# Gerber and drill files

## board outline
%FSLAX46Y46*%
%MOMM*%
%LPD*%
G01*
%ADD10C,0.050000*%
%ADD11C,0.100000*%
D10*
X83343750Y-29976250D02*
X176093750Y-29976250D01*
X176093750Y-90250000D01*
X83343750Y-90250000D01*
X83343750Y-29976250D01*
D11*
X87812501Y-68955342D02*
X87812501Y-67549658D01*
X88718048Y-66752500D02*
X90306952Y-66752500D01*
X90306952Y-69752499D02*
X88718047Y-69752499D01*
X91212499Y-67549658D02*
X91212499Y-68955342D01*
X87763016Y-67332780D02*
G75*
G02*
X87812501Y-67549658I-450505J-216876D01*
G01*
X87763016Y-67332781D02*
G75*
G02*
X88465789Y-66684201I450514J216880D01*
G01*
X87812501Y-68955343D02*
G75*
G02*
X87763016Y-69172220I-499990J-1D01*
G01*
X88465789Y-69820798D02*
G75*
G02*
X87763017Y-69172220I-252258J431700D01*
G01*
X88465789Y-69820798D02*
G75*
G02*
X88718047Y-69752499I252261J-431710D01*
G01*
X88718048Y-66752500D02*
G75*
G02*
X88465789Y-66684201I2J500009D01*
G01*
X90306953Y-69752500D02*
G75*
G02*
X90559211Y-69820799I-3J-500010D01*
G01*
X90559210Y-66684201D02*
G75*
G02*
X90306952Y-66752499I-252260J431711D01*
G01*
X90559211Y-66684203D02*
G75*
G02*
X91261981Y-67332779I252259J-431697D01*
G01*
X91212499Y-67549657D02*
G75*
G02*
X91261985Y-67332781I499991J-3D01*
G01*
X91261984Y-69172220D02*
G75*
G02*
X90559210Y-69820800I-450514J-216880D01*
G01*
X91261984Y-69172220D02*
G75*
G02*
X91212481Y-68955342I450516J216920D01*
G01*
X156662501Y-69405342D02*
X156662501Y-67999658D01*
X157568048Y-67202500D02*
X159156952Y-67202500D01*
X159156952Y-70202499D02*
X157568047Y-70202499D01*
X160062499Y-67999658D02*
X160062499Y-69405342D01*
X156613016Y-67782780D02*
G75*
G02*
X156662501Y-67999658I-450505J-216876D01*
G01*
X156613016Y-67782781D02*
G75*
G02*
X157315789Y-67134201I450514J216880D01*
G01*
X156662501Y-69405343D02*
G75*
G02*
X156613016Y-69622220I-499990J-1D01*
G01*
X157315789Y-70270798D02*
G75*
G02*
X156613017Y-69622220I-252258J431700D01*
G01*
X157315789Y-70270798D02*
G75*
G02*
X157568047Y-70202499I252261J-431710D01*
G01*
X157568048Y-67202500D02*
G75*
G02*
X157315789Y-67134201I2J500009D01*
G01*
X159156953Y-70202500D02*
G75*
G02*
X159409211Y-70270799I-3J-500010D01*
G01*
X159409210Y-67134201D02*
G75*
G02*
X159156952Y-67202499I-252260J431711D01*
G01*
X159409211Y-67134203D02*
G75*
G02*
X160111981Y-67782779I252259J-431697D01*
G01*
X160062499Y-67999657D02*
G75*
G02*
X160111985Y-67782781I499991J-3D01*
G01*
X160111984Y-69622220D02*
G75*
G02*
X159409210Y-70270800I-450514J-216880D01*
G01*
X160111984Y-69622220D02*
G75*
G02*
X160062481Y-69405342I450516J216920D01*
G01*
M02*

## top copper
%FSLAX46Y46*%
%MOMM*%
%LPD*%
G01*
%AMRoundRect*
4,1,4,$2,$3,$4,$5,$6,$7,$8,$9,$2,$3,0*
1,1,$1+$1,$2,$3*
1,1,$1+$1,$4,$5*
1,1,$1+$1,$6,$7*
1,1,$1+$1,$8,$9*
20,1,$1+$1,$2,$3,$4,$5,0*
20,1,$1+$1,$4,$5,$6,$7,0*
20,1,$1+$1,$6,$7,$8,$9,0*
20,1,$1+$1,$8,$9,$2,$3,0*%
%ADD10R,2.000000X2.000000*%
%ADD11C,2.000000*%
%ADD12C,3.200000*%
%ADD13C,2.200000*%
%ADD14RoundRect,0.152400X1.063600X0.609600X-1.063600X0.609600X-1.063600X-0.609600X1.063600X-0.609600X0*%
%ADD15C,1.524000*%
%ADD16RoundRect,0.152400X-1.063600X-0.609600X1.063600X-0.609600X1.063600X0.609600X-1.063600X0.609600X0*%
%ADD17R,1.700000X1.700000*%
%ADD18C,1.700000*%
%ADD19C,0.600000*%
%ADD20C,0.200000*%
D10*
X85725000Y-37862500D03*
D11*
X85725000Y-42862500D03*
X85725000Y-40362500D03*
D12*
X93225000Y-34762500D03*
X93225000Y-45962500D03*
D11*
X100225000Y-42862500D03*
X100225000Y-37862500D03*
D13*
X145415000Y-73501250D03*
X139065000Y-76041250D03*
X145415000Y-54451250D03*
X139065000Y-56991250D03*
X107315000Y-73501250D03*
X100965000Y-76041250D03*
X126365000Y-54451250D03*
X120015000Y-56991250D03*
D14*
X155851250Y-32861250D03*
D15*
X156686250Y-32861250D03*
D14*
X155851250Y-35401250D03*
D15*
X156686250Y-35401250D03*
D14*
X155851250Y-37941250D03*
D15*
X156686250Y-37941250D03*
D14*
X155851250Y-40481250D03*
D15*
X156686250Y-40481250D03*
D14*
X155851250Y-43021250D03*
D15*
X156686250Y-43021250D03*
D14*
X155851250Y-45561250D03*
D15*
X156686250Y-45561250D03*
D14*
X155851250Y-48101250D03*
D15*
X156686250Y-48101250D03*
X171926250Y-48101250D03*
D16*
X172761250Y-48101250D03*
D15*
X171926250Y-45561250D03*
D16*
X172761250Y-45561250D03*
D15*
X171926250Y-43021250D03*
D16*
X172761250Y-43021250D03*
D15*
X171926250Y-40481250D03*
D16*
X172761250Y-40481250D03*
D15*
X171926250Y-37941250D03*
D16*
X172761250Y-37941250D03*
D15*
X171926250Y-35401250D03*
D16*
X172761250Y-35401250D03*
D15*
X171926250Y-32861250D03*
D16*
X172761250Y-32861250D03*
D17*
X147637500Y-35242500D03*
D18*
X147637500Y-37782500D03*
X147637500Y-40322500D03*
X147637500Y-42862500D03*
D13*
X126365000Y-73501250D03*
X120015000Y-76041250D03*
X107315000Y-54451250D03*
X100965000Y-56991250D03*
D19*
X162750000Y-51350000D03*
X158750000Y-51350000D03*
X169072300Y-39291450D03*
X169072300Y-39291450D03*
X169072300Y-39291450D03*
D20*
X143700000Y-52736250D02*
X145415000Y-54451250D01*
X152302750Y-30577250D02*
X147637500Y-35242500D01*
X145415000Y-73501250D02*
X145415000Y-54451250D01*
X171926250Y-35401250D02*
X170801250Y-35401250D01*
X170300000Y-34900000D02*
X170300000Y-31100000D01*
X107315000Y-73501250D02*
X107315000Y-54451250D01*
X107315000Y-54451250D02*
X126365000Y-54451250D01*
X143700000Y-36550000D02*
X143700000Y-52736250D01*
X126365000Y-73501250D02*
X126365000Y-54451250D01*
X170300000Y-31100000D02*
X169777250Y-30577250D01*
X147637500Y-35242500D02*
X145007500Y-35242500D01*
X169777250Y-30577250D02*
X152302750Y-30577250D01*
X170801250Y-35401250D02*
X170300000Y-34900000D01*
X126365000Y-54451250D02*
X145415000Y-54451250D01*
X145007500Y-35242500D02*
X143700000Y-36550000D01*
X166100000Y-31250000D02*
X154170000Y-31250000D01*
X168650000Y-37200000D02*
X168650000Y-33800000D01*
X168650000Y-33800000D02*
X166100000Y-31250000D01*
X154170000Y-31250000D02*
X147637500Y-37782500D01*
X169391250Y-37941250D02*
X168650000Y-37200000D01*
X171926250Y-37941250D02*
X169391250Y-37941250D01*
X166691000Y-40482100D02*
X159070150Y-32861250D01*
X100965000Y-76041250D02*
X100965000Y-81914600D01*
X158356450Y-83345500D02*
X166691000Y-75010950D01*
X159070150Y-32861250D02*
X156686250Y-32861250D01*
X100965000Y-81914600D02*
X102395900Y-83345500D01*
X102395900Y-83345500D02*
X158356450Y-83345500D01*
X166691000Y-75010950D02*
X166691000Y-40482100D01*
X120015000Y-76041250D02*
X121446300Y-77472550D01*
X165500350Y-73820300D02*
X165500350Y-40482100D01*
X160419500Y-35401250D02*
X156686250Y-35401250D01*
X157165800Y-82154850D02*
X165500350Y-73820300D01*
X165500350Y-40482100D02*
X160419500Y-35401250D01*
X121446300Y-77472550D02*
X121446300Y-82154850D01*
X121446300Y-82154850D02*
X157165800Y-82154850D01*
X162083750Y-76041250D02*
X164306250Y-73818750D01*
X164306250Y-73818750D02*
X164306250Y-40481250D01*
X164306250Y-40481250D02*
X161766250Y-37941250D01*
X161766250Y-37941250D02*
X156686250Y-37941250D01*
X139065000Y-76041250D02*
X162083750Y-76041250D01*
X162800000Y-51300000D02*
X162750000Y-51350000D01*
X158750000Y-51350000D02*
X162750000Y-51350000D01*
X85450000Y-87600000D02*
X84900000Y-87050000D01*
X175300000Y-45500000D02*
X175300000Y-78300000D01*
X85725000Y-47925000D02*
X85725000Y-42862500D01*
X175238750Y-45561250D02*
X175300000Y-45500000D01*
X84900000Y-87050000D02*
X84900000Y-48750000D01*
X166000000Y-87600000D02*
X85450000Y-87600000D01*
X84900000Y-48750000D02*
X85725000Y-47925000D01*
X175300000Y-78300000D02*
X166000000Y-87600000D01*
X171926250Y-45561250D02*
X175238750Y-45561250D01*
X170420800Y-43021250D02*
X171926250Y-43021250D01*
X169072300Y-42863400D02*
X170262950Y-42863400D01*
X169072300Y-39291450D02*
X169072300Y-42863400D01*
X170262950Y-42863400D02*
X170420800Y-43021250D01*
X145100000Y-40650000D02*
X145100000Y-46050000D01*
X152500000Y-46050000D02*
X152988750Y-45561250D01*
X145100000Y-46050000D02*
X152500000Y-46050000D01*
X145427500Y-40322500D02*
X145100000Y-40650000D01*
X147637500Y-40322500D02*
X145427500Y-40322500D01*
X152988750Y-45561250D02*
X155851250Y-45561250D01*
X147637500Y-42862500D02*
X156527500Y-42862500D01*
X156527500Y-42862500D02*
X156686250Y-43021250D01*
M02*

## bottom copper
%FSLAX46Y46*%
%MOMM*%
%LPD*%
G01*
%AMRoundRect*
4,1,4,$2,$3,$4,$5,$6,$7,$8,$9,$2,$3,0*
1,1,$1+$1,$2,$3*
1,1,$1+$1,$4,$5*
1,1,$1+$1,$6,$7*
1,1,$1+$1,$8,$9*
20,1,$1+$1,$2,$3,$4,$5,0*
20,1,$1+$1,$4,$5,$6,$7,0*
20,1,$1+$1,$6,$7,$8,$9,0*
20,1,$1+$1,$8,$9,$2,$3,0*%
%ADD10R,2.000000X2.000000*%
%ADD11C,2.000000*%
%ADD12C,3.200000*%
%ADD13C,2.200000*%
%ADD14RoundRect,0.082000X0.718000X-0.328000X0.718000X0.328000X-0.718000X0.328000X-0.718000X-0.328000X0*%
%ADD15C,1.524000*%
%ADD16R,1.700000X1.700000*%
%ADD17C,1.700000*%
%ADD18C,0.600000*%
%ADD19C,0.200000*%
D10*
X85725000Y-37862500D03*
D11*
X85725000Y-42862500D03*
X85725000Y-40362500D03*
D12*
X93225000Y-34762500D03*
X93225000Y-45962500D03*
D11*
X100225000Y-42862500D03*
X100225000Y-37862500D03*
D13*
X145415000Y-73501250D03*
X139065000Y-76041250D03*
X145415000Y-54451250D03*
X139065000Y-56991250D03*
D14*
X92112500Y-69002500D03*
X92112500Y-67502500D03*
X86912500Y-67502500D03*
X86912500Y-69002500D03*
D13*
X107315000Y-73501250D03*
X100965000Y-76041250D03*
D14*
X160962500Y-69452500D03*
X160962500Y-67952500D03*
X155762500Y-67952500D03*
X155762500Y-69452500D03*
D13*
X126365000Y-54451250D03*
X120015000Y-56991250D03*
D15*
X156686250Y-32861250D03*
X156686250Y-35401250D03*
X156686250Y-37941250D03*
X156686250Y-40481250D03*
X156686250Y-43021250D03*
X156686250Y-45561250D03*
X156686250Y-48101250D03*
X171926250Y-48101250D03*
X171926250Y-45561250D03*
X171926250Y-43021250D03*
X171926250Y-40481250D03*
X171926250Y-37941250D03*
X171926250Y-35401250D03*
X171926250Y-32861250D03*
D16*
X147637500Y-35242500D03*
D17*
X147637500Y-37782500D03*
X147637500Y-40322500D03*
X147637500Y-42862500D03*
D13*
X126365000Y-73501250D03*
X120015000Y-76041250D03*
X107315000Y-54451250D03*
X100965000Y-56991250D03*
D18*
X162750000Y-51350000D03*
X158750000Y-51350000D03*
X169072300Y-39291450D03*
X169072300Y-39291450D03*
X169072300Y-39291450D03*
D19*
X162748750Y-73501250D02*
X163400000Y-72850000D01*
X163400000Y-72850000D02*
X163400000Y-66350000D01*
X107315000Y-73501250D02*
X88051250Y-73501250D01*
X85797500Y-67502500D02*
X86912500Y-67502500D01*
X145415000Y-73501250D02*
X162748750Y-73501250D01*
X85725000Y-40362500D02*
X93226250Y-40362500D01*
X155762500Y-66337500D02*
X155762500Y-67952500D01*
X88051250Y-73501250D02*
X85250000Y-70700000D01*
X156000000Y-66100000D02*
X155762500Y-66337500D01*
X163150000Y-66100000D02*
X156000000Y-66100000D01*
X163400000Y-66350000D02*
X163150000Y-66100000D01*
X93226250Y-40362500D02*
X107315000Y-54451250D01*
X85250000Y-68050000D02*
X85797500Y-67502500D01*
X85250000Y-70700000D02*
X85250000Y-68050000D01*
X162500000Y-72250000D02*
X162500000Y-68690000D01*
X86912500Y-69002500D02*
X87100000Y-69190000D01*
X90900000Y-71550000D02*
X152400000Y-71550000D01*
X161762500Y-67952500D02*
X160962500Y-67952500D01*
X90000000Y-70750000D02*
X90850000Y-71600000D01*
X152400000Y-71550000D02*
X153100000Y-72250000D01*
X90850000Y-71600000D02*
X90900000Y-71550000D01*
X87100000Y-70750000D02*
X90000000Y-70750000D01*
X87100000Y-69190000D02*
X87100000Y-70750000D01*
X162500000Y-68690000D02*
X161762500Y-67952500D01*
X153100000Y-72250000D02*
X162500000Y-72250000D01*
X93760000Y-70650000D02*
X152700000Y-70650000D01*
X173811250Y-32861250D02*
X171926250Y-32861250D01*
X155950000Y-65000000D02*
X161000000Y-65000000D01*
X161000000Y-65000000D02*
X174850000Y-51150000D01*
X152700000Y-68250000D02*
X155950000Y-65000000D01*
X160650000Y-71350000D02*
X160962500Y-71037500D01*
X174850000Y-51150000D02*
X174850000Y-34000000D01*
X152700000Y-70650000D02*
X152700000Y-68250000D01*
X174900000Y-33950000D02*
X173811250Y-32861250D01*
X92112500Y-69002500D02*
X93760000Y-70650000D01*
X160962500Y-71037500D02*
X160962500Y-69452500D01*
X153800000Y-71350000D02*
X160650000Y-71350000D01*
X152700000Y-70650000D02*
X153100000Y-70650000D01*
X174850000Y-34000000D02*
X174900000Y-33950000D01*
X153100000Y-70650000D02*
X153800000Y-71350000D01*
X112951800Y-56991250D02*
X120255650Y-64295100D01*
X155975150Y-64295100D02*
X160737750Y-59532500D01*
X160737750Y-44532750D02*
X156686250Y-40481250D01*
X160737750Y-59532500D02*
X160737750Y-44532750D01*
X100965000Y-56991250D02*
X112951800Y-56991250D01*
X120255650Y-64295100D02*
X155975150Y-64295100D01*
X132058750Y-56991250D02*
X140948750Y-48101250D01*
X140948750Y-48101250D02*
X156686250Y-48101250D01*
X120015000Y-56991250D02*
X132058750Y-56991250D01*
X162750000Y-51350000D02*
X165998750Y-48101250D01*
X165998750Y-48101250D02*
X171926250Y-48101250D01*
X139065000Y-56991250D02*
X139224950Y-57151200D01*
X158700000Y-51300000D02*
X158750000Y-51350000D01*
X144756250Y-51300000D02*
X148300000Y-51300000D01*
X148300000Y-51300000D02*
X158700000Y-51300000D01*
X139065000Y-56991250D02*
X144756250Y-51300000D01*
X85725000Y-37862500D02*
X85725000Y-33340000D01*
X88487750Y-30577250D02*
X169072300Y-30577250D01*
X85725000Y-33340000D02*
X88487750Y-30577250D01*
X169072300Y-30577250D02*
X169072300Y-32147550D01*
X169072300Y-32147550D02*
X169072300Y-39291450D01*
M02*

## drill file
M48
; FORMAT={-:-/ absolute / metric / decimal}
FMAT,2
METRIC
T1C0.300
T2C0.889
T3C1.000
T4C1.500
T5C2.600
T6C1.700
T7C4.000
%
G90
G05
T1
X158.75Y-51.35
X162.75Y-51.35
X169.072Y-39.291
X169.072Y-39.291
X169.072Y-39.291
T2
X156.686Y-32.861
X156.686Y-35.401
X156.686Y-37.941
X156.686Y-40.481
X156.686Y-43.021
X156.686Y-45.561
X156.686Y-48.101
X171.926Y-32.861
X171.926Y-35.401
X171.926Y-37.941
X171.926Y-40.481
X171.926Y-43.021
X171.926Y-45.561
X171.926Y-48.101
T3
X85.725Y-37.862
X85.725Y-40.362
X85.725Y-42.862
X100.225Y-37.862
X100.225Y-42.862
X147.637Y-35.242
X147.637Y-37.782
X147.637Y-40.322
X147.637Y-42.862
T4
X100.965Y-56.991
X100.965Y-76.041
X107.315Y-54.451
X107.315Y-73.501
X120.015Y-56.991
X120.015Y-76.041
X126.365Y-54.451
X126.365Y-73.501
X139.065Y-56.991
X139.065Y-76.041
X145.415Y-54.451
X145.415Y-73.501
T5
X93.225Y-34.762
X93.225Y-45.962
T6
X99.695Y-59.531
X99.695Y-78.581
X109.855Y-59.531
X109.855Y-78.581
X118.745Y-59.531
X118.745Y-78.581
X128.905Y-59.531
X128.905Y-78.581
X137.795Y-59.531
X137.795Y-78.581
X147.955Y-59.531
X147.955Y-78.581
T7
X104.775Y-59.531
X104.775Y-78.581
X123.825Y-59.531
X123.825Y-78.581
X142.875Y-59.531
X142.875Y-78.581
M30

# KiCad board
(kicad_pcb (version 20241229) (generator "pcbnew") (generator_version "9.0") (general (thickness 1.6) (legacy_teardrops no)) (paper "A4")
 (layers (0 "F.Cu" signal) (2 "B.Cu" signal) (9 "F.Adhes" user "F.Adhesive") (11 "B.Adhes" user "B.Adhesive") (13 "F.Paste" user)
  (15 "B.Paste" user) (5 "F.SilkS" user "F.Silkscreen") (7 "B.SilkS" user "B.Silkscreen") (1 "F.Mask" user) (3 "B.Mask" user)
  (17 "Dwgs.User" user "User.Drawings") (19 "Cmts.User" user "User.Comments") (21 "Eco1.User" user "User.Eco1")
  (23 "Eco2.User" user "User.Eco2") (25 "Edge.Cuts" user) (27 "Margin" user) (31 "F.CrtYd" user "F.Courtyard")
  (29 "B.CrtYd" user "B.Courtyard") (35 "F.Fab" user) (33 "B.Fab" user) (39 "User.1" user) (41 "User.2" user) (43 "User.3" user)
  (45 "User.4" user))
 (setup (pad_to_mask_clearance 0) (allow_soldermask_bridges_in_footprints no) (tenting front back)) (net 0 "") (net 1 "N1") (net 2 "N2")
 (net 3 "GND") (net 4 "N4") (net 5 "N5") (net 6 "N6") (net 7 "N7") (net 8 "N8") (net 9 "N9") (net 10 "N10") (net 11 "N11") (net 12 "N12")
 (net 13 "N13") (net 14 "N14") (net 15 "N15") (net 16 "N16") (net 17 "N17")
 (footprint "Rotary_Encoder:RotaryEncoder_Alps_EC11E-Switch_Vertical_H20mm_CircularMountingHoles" (layer "F.Cu") (at 85.725 37.8625)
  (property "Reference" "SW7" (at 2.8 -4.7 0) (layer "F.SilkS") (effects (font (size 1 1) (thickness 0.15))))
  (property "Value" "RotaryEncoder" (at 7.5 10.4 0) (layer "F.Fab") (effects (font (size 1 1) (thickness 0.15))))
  (pad "A" thru_hole rect (at 0 0) (size 2 2) (drill 1) (layers "*.Cu" "*.Mask") (remove_unused_layers no) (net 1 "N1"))
  (pad "B" thru_hole circle (at 0 5) (size 2 2) (drill 1) (layers "*.Cu" "*.Mask") (remove_unused_layers no) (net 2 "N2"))
  (pad "C" thru_hole circle (at 0 2.5) (size 2 2) (drill 1) (layers "*.Cu" "*.Mask") (remove_unused_layers no) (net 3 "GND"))
  (pad "MP" thru_hole circle (at 7.5 -3.1) (size 3.2 3.2) (drill 2.6) (layers "*.Cu" "*.Mask") (remove_unused_layers no))
  (pad "MP" thru_hole circle (at 7.5 8.1) (size 3.2 3.2) (drill 2.6) (layers "*.Cu" "*.Mask") (remove_unused_layers no))
  (pad "S1" thru_hole circle (at 14.5 5) (size 2 2) (drill 1) (layers "*.Cu" "*.Mask") (remove_unused_layers no))
  (pad "S2" thru_hole circle (at 14.5 0) (size 2 2) (drill 1) (layers "*.Cu" "*.Mask") (remove_unused_layers no)))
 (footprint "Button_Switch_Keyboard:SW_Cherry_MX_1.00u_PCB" (layer "F.Cu") (at 145.415 73.50125)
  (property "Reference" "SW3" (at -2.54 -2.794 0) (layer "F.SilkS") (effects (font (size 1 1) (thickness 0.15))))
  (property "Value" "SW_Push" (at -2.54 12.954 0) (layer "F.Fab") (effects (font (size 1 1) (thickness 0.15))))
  (pad "" np_thru_hole circle (at -7.62 5.08) (size 1.7 1.7) (drill 1.7) (layers "*.Cu" "*.Mask"))
  (pad "" np_thru_hole circle (at -2.54 5.08) (size 4 4) (drill 4) (layers "*.Cu" "*.Mask"))
  (pad "" np_thru_hole circle (at 2.54 5.08) (size 1.7 1.7) (drill 1.7) (layers "*.Cu" "*.Mask"))
  (pad "1" thru_hole circle (at 0 0) (size 2.2 2.2) (drill 1.5) (layers "*.Cu" "*.Mask") (remove_unused_layers no) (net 3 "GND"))
  (pad "2" thru_hole circle (at -6.35 2.54) (size 2.2 2.2) (drill 1.5) (layers "*.Cu" "*.Mask") (remove_unused_layers no) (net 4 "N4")))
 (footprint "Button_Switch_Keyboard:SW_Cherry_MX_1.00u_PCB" (layer "F.Cu") (at 145.415 54.45125)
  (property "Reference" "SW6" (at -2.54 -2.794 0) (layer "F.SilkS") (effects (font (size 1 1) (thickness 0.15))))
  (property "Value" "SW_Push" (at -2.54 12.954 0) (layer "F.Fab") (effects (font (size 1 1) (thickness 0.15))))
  (pad "" np_thru_hole circle (at -7.62 5.08) (size 1.7 1.7) (drill 1.7) (layers "*.Cu" "*.Mask"))
  (pad "" np_thru_hole circle (at -2.54 5.08) (size 4 4) (drill 4) (layers "*.Cu" "*.Mask"))
  (pad "" np_thru_hole circle (at 2.54 5.08) (size 1.7 1.7) (drill 1.7) (layers "*.Cu" "*.Mask"))
  (pad "1" thru_hole circle (at 0 0) (size 2.2 2.2) (drill 1.5) (layers "*.Cu" "*.Mask") (remove_unused_layers no) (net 3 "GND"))
  (pad "2" thru_hole circle (at -6.35 2.54) (size 2.2 2.2) (drill 1.5) (layers "*.Cu" "*.Mask") (remove_unused_layers no) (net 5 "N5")))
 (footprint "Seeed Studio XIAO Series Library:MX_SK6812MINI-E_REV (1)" (layer "F.Cu") (at 89.5125 63.1725)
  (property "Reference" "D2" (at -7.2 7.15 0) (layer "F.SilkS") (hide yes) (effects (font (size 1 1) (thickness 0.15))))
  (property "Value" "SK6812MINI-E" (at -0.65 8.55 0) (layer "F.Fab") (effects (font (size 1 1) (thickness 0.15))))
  (fp_line (start -1.699999 5.782842) (end -1.699999 4.377158) (stroke (width 0.1) (type solid)) (layer "Edge.Cuts"))
  (fp_line (start -0.794452 3.58) (end 0.794452 3.58) (stroke (width 0.1) (type solid)) (layer "Edge.Cuts"))
  (fp_line (start 0.794452 6.579999) (end -0.794453 6.579999) (stroke (width 0.1) (type solid)) (layer "Edge.Cuts"))
  (fp_line (start 1.699999 4.377158) (end 1.699999 5.782842) (stroke (width 0.1) (type solid)) (layer "Edge.Cuts"))
  (fp_arc (start -1.749484 4.16028) (mid -1.712527 4.265932) (end -1.699999 4.377158) (stroke (width 0.1) (type solid)) (layer "Edge.Cuts"))
  (fp_arc (start -1.749484 4.160281) (mid -1.638072 3.575965) (end -1.046711 3.511701) (stroke (width 0.1) (type solid)) (layer "Edge.Cuts"))
  (fp_arc (start -1.699999 5.782843) (mid -1.712527 5.894068) (end -1.749484 5.99972) (stroke (width 0.1) (type solid)) (layer "Edge.Cuts"))
  (fp_arc (start -1.046711 6.648298) (mid -1.638071 6.584034) (end -1.749484 5.99972) (stroke (width 0.1) (type solid)) (layer "Edge.Cuts"))
  (fp_arc (start -1.046711 6.648298) (mid -0.925123 6.597376) (end -0.794453 6.579999) (stroke (width 0.1) (type solid)) (layer "Edge.Cuts"))
  (fp_arc (start -0.794452 3.58) (mid -0.925123 3.562623) (end -1.046711 3.511701) (stroke (width 0.1) (type solid)) (layer "Edge.Cuts"))
  (fp_arc (start 0.794453 6.58) (mid 0.925123 6.597377) (end 1.046711 6.648299) (stroke (width 0.1) (type solid)) (layer "Edge.Cuts"))
  (fp_arc (start 1.04671 3.511701) (mid 0.925122 3.562623) (end 0.794452 3.58) (stroke (width 0.1) (type solid)) (layer "Edge.Cuts"))
  (fp_arc (start 1.046711 3.511703) (mid 1.63807 3.575966) (end 1.749484 4.16028) (stroke (width 0.1) (type solid)) (layer "Edge.Cuts"))
  (fp_arc (start 1.699999 4.377157) (mid 1.712527 4.265932) (end 1.749484 4.16028) (stroke (width 0.1) (type solid)) (layer "Edge.Cuts"))
  (fp_arc (start 1.749484 5.99972) (mid 1.638071 6.584035) (end 1.046711 6.648299) (stroke (width 0.1) (type solid)) (layer "Edge.Cuts"))
  (fp_arc (start 1.749484 5.99972) (mid 1.712527 5.894068) (end 1.699999 5.782842) (stroke (width 0.1) (type solid)) (layer "Edge.Cuts"))
  (pad "1" smd roundrect (at 2.6 5.83 90) (size 0.82 1.6) (layers "B.Cu" "B.Mask" "B.Paste") (roundrect_rratio 0.1) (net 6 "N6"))
  (pad "2" smd roundrect (at 2.6 4.33 90) (size 0.82 1.6) (layers "B.Cu" "B.Mask" "B.Paste") (roundrect_rratio 0.1) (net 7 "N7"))
  (pad "3" smd roundrect (at -2.6 4.33 90) (size 0.82 1.6) (layers "B.Cu" "B.Mask" "B.Paste") (roundrect_rratio 0.1) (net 3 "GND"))
  (pad "4" smd roundrect (at -2.6 5.83 90) (size 0.82 1.6) (layers "B.Cu" "B.Mask" "B.Paste") (roundrect_rratio 0.1) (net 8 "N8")))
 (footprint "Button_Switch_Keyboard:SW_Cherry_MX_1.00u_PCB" (layer "F.Cu") (at 107.315 73.50125)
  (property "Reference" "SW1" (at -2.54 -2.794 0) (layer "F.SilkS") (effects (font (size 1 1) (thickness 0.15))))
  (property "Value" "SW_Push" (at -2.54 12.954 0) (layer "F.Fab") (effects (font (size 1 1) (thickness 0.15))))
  (pad "" np_thru_hole circle (at -7.62 5.08) (size 1.7 1.7) (drill 1.7) (layers "*.Cu" "*.Mask"))
  (pad "" np_thru_hole circle (at -2.54 5.08) (size 4 4) (drill 4) (layers "*.Cu" "*.Mask"))
  (pad "" np_thru_hole circle (at 2.54 5.08) (size 1.7 1.7) (drill 1.7) (layers "*.Cu" "*.Mask"))
  (pad "1" thru_hole circle (at 0 0) (size 2.2 2.2) (drill 1.5) (layers "*.Cu" "*.Mask") (remove_unused_layers no) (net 3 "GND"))
  (pad "2" thru_hole circle (at -6.35 2.54) (size 2.2 2.2) (drill 1.5) (layers "*.Cu" "*.Mask") (remove_unused_layers no) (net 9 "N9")))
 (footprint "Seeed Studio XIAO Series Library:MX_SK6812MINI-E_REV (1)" (layer "F.Cu") (at 158.3625 63.6225)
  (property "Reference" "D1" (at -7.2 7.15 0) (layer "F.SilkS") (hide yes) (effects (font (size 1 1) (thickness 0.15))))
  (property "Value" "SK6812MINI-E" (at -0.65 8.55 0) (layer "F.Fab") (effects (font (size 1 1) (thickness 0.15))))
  (fp_line (start -1.699999 5.782842) (end -1.699999 4.377158) (stroke (width 0.1) (type solid)) (layer "Edge.Cuts"))
  (fp_line (start -0.794452 3.58) (end 0.794452 3.58) (stroke (width 0.1) (type solid)) (layer "Edge.Cuts"))
  (fp_line (start 0.794452 6.579999) (end -0.794453 6.579999) (stroke (width 0.1) (type solid)) (layer "Edge.Cuts"))
  (fp_line (start 1.699999 4.377158) (end 1.699999 5.782842) (stroke (width 0.1) (type solid)) (layer "Edge.Cuts"))
  (fp_arc (start -1.749484 4.16028) (mid -1.712527 4.265932) (end -1.699999 4.377158) (stroke (width 0.1) (type solid)) (layer "Edge.Cuts"))
  (fp_arc (start -1.749484 4.160281) (mid -1.638072 3.575965) (end -1.046711 3.511701) (stroke (width 0.1) (type solid)) (layer "Edge.Cuts"))
  (fp_arc (start -1.699999 5.782843) (mid -1.712527 5.894068) (end -1.749484 5.99972) (stroke (width 0.1) (type solid)) (layer "Edge.Cuts"))
  (fp_arc (start -1.046711 6.648298) (mid -1.638071 6.584034) (end -1.749484 5.99972) (stroke (width 0.1) (type solid)) (layer "Edge.Cuts"))
  (fp_arc (start -1.046711 6.648298) (mid -0.925123 6.597376) (end -0.794453 6.579999) (stroke (width 0.1) (type solid)) (layer "Edge.Cuts"))
  (fp_arc (start -0.794452 3.58) (mid -0.925123 3.562623) (end -1.046711 3.511701) (stroke (width 0.1) (type solid)) (layer "Edge.Cuts"))
  (fp_arc (start 0.794453 6.58) (mid 0.925123 6.597377) (end 1.046711 6.648299) (stroke (width 0.1) (type solid)) (layer "Edge.Cuts"))
  (fp_arc (start 1.04671 3.511701) (mid 0.925122 3.562623) (end 0.794452 3.58) (stroke (width 0.1) (type solid)) (layer "Edge.Cuts"))
  (fp_arc (start 1.046711 3.511703) (mid 1.63807 3.575966) (end 1.749484 4.16028) (stroke (width 0.1) (type solid)) (layer "Edge.Cuts"))
  (fp_arc (start 1.699999 4.377157) (mid 1.712527 4.265932) (end 1.749484 4.16028) (stroke (width 0.1) (type solid)) (layer "Edge.Cuts"))
  (fp_arc (start 1.749484 5.99972) (mid 1.638071 6.584035) (end 1.046711 6.648299) (stroke (width 0.1) (type solid)) (layer "Edge.Cuts"))
  (fp_arc (start 1.749484 5.99972) (mid 1.712527 5.894068) (end 1.699999 5.782842) (stroke (width 0.1) (type solid)) (layer "Edge.Cuts"))
  (pad "1" smd roundrect (at 2.6 5.83 90) (size 0.82 1.6) (layers "B.Cu" "B.Mask" "B.Paste") (roundrect_rratio 0.1) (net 6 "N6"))
  (pad "2" smd roundrect (at 2.6 4.33 90) (size 0.82 1.6) (layers "B.Cu" "B.Mask" "B.Paste") (roundrect_rratio 0.1) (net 8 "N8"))
  (pad "3" smd roundrect (at -2.6 4.33 90) (size 0.82 1.6) (layers "B.Cu" "B.Mask" "B.Paste") (roundrect_rratio 0.1) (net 3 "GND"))
  (pad "4" smd roundrect (at -2.6 5.83 90) (size 0.82 1.6) (layers "B.Cu" "B.Mask" "B.Paste") (roundrect_rratio 0.1) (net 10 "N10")))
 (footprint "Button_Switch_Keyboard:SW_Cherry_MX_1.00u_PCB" (layer "F.Cu") (at 126.365 54.45125)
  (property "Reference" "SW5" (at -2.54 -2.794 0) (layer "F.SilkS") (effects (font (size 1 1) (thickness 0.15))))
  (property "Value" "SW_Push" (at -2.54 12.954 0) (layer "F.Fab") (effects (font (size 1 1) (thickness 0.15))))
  (pad "" np_thru_hole circle (at -7.62 5.08) (size 1.7 1.7) (drill 1.7) (layers "*.Cu" "*.Mask"))
  (pad "" np_thru_hole circle (at -2.54 5.08) (size 4 4) (drill 4) (layers "*.Cu" "*.Mask"))
  (pad "" np_thru_hole circle (at 2.54 5.08) (size 1.7 1.7) (drill 1.7) (layers "*.Cu" "*.Mask"))
  (pad "1" thru_hole circle (at 0 0) (size 2.2 2.2) (drill 1.5) (layers "*.Cu" "*.Mask") (remove_unused_layers no) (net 3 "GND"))
  (pad "2" thru_hole circle (at -6.35 2.54) (size 2.2 2.2) (drill 1.5) (layers "*.Cu" "*.Mask") (remove_unused_layers no) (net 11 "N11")))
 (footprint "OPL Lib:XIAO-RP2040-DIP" (layer "F.Cu") (at 164.30625 40.48125)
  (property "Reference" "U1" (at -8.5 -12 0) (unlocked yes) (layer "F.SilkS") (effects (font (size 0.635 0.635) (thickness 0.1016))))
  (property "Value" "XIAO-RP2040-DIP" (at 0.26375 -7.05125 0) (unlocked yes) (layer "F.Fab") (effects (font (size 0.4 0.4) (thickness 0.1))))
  (pad "1" smd roundrect (at -8.455 -7.62 180) (size 2.432 1.524) (layers "F.Cu" "F.Mask") (roundrect_rratio 0.1) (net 9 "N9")
   (thermal_bridge_angle 45))
  (pad "1" thru_hole circle (at -7.62 -7.62 180) (size 1.524 1.524) (drill 0.889) (layers "*.Cu" "*.Mask") (remove_unused_layers no)
   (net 9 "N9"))
  (pad "2" smd roundrect (at -8.455 -5.08 180) (size 2.432 1.524) (layers "F.Cu" "F.Mask") (roundrect_rratio 0.1) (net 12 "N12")
   (thermal_bridge_angle 45))
  (pad "2" thru_hole circle (at -7.62 -5.08 180) (size 1.524 1.524) (drill 0.889) (layers "*.Cu" "*.Mask") (remove_unused_layers no)
   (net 12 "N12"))
  (pad "3" smd roundrect (at -8.455 -2.54 180) (size 2.432 1.524) (layers "F.Cu" "F.Mask") (roundrect_rratio 0.1) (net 4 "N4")
   (thermal_bridge_angle 45))
  (pad "3" thru_hole circle (at -7.62 -2.54 180) (size 1.524 1.524) (drill 0.889) (layers "*.Cu" "*.Mask") (remove_unused_layers no)
   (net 4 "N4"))
  (pad "4" smd roundrect (at -8.455 0 180) (size 2.432 1.524) (layers "F.Cu" "F.Mask") (roundrect_rratio 0.1) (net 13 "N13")
   (thermal_bridge_angle 45))
  (pad "4" thru_hole circle (at -7.62 0 180) (size 1.524 1.524) (drill 0.889) (layers "*.Cu" "*.Mask") (remove_unused_layers no)
   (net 13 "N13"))
  (pad "5" smd roundrect (at -8.455 2.54 180) (size 2.432 1.524) (layers "F.Cu" "F.Mask") (roundrect_rratio 0.1) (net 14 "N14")
   (thermal_bridge_angle 45))
  (pad "5" thru_hole circle (at -7.62 2.54 180) (size 1.524 1.524) (drill 0.889) (layers "*.Cu" "*.Mask") (remove_unused_layers no)
   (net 14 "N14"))
  (pad "6" smd roundrect (at -8.455 5.08 180) (size 2.432 1.524) (layers "F.Cu" "F.Mask") (roundrect_rratio 0.1) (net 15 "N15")
   (thermal_bridge_angle 45))
  (pad "6" thru_hole circle (at -7.62 5.08 180) (size 1.524 1.524) (drill 0.889) (layers "*.Cu" "*.Mask") (remove_unused_layers no)
   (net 15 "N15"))
  (pad "7" smd roundrect (at -8.455 7.62 180) (size 2.432 1.524) (layers "F.Cu" "F.Mask") (roundrect_rratio 0.1) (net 11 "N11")
   (thermal_bridge_angle 45))
  (pad "7" thru_hole circle (at -7.62 7.62 180) (size 1.524 1.524) (drill 0.889) (layers "*.Cu" "*.Mask") (remove_unused_layers no)
   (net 11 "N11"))
  (pad "8" thru_hole circle (at 7.62 7.62) (size 1.524 1.524) (drill 0.889) (layers "*.Cu" "*.Mask") (remove_unused_layers no) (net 5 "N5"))
  (pad "8" smd roundrect (at 8.455 7.62) (size 2.432 1.524) (layers "F.Cu" "F.Mask") (roundrect_rratio 0.1) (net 5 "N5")
   (thermal_bridge_angle 45))
  (pad "9" thru_hole circle (at 7.62 5.08) (size 1.524 1.524) (drill 0.889) (layers "*.Cu" "*.Mask") (remove_unused_layers no) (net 2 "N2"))
  (pad "9" smd roundrect (at 8.455 5.08) (size 2.432 1.524) (layers "F.Cu" "F.Mask") (roundrect_rratio 0.1) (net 2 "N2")
   (thermal_bridge_angle 45))
  (pad "10" thru_hole circle (at 7.62 2.54) (size 1.524 1.524) (drill 0.889) (layers "*.Cu" "*.Mask") (remove_unused_layers no) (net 1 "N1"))
  (pad "10" smd roundrect (at 8.455 2.54) (size 2.432 1.524) (layers "F.Cu" "F.Mask") (roundrect_rratio 0.1) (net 1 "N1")
   (thermal_bridge_angle 45))
  (pad "11" thru_hole circle (at 7.62 0) (size 1.524 1.524) (drill 0.889) (layers "*.Cu" "*.Mask") (remove_unused_layers no) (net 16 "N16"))
  (pad "11" smd roundrect (at 8.455 0) (size 2.432 1.524) (layers "F.Cu" "F.Mask") (roundrect_rratio 0.1) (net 16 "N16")
   (thermal_bridge_angle 45))
  (pad "12" thru_hole circle (at 7.62 -2.54) (size 1.524 1.524) (drill 0.889) (layers "*.Cu" "*.Mask") (remove_unused_layers no)
   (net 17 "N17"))
  (pad "12" smd roundrect (at 8.455 -2.54) (size 2.432 1.524) (layers "F.Cu" "F.Mask") (roundrect_rratio 0.1) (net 17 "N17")
   (thermal_bridge_angle 45))
  (pad "13" thru_hole circle (at 7.62 -5.08) (size 1.524 1.524) (drill 0.889) (layers "*.Cu" "*.Mask") (remove_unused_layers no)
   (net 3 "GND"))
  (pad "13" smd roundrect (at 8.455 -5.08) (size 2.432 1.524) (layers "F.Cu" "F.Mask") (roundrect_rratio 0.1) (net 3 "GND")
   (thermal_bridge_angle 45))
  (pad "14" thru_hole circle (at 7.62 -7.62) (size 1.524 1.524) (drill 0.889) (layers "*.Cu" "*.Mask") (remove_unused_layers no)
   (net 6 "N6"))
  (pad "14" smd roundrect (at 8.455 -7.62) (size 2.432 1.524) (layers "F.Cu" "F.Mask") (roundrect_rratio 0.1) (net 6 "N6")
   (thermal_bridge_angle 45)))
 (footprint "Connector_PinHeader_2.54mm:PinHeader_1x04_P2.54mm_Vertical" (layer "F.Cu") (at 147.6375 35.2425)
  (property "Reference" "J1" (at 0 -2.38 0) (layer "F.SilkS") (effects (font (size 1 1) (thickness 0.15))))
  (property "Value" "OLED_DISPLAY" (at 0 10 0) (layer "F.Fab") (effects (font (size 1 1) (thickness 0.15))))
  (pad "1" thru_hole rect (at 0 0) (size 1.7 1.7) (drill 1) (layers "*.Cu" "*.Mask") (remove_unused_layers no) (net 3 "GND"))
  (pad "2" thru_hole circle (at 0 2.54) (size 1.7 1.7) (drill 1) (layers "*.Cu" "*.Mask") (remove_unused_layers no) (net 17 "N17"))
  (pad "3" thru_hole circle (at 0 5.08) (size 1.7 1.7) (drill 1) (layers "*.Cu" "*.Mask") (remove_unused_layers no) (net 15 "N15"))
  (pad "4" thru_hole circle (at 0 7.62) (size 1.7 1.7) (drill 1) (layers "*.Cu" "*.Mask") (remove_unused_layers no) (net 14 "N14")))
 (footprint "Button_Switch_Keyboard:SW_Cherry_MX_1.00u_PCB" (layer "F.Cu") (at 126.365 73.50125)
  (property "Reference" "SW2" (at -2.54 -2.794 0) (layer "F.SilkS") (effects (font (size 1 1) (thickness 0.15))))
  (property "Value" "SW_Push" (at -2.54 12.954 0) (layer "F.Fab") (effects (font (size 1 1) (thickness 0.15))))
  (pad "" np_thru_hole circle (at -7.62 5.08) (size 1.7 1.7) (drill 1.7) (layers "*.Cu" "*.Mask"))
  (pad "" np_thru_hole circle (at -2.54 5.08) (size 4 4) (drill 4) (layers "*.Cu" "*.Mask"))
  (pad "" np_thru_hole circle (at 2.54 5.08) (size 1.7 1.7) (drill 1.7) (layers "*.Cu" "*.Mask"))
  (pad "1" thru_hole circle (at 0 0) (size 2.2 2.2) (drill 1.5) (layers "*.Cu" "*.Mask") (remove_unused_layers no) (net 3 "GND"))
  (pad "2" thru_hole circle (at -6.35 2.54) (size 2.2 2.2) (drill 1.5) (layers "*.Cu" "*.Mask") (remove_unused_layers no) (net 12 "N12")))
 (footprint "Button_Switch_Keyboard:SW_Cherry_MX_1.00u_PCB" (layer "F.Cu") (at 107.315 54.45125)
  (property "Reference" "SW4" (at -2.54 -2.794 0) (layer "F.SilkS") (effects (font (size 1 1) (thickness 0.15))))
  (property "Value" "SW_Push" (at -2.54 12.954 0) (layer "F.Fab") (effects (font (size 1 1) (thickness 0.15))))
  (pad "" np_thru_hole circle (at -7.62 5.08) (size 1.7 1.7) (drill 1.7) (layers "*.Cu" "*.Mask"))
  (pad "" np_thru_hole circle (at -2.54 5.08) (size 4 4) (drill 4) (layers "*.Cu" "*.Mask"))
  (pad "" np_thru_hole circle (at 2.54 5.08) (size 1.7 1.7) (drill 1.7) (layers "*.Cu" "*.Mask"))
  (pad "1" thru_hole circle (at 0 0) (size 2.2 2.2) (drill 1.5) (layers "*.Cu" "*.Mask") (remove_unused_layers no) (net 3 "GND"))
  (pad "2" thru_hole circle (at -6.35 2.54) (size 2.2 2.2) (drill 1.5) (layers "*.Cu" "*.Mask") (remove_unused_layers no) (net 13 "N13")))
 (gr_rect (start 83.34375 29.97625) (end 176.09375 90.25) (stroke (width 0.05) (type default)) (fill no) (layer "Edge.Cuts"))
 (segment (start 143.7 52.73625) (end 145.415 54.45125) (width 0.2) (layer "F.Cu") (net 3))
 (segment (start 152.30275 30.57725) (end 147.6375 35.2425) (width 0.2) (layer "F.Cu") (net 3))
 (segment (start 145.415 73.50125) (end 145.415 54.45125) (width 0.2) (layer "F.Cu") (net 3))
 (segment (start 171.92625 35.40125) (end 170.80125 35.40125) (width 0.2) (layer "F.Cu") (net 3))
 (segment (start 170.3 34.9) (end 170.3 31.1) (width 0.2) (layer "F.Cu") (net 3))
 (segment (start 107.315 73.50125) (end 107.315 54.45125) (width 0.2) (layer "F.Cu") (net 3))
 (segment (start 107.315 54.45125) (end 126.365 54.45125) (width 0.2) (layer "F.Cu") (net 3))
 (segment (start 143.7 36.55) (end 143.7 52.73625) (width 0.2) (layer "F.Cu") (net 3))
 (segment (start 126.365 73.50125) (end 126.365 54.45125) (width 0.2) (layer "F.Cu") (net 3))
 (segment (start 170.3 31.1) (end 169.77725 30.57725) (width 0.2) (layer "F.Cu") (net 3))
 (segment (start 147.6375 35.2425) (end 145.0075 35.2425) (width 0.2) (layer "F.Cu") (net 3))
 (segment (start 169.77725 30.57725) (end 152.30275 30.57725) (width 0.2) (layer "F.Cu") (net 3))
 (segment (start 170.80125 35.40125) (end 170.3 34.9) (width 0.2) (layer "F.Cu") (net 3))
 (segment (start 126.365 54.45125) (end 145.415 54.45125) (width 0.2) (layer "F.Cu") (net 3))
 (segment (start 145.0075 35.2425) (end 143.7 36.55) (width 0.2) (layer "F.Cu") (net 3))
 (segment (start 162.74875 73.50125) (end 163.4 72.85) (width 0.2) (layer "B.Cu") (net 3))
 (segment (start 163.4 72.85) (end 163.4 66.35) (width 0.2) (layer "B.Cu") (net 3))
 (segment (start 107.315 73.50125) (end 88.05125 73.50125) (width 0.2) (layer "B.Cu") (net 3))
 (segment (start 85.7975 67.5025) (end 86.9125 67.5025) (width 0.2) (layer "B.Cu") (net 3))
 (segment (start 145.415 73.50125) (end 162.74875 73.50125) (width 0.2) (layer "B.Cu") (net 3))
 (segment (start 85.725 40.3625) (end 93.22625 40.3625) (width 0.2) (layer "B.Cu") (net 3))
 (segment (start 155.7625 66.3375) (end 155.7625 67.9525) (width 0.2) (layer "B.Cu") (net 3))
 (segment (start 88.05125 73.50125) (end 85.25 70.7) (width 0.2) (layer "B.Cu") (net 3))
 (segment (start 156 66.1) (end 155.7625 66.3375) (width 0.2) (layer "B.Cu") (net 3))
 (segment (start 163.15 66.1) (end 156 66.1) (width 0.2) (layer "B.Cu") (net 3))
 (segment (start 163.4 66.35) (end 163.15 66.1) (width 0.2) (layer "B.Cu") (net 3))
 (segment (start 93.22625 40.3625) (end 107.315 54.45125) (width 0.2) (layer "B.Cu") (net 3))
 (segment (start 85.25 68.05) (end 85.7975 67.5025) (width 0.2) (layer "B.Cu") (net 3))
 (segment (start 85.25 70.7) (end 85.25 68.05) (width 0.2) (layer "B.Cu") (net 3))
 (segment (start 162.5 72.25) (end 162.5 68.69) (width 0.2) (layer "B.Cu") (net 8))
 (segment (start 86.9125 69.0025) (end 87.1 69.19) (width 0.2) (layer "B.Cu") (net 8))
 (segment (start 90.9 71.55) (end 152.4 71.55) (width 0.2) (layer "B.Cu") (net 8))
 (segment (start 161.7625 67.9525) (end 160.9625 67.9525) (width 0.2) (layer "B.Cu") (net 8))
 (segment (start 90 70.75) (end 90.85 71.6) (width 0.2) (layer "B.Cu") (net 8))
 (segment (start 152.4 71.55) (end 153.1 72.25) (width 0.2) (layer "B.Cu") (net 8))
 (segment (start 90.85 71.6) (end 90.9 71.55) (width 0.2) (layer "B.Cu") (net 8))
 (segment (start 87.1 70.75) (end 90 70.75) (width 0.2) (layer "B.Cu") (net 8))
 (segment (start 87.1 69.19) (end 87.1 70.75) (width 0.2) (layer "B.Cu") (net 8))
 (segment (start 162.5 68.69) (end 161.7625 67.9525) (width 0.2) (layer "B.Cu") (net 8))
 (segment (start 153.1 72.25) (end 162.5 72.25) (width 0.2) (layer "B.Cu") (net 8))
 (segment (start 93.76 70.65) (end 152.7 70.65) (width 0.2) (layer "B.Cu") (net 6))
 (segment (start 173.81125 32.86125) (end 171.92625 32.86125) (width 0.2) (layer "B.Cu") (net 6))
 (segment (start 155.95 65) (end 161 65) (width 0.2) (layer "B.Cu") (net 6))
 (segment (start 161 65) (end 174.85 51.15) (width 0.2) (layer "B.Cu") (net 6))
 (segment (start 152.7 68.25) (end 155.95 65) (width 0.2) (layer "B.Cu") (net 6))
 (segment (start 160.65 71.35) (end 160.9625 71.0375) (width 0.2) (layer "B.Cu") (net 6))
 (segment (start 174.85 51.15) (end 174.85 34) (width 0.2) (layer "B.Cu") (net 6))
 (segment (start 152.7 70.65) (end 152.7 68.25) (width 0.2) (layer "B.Cu") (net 6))
 (segment (start 174.9 33.95) (end 173.81125 32.86125) (width 0.2) (layer "B.Cu") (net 6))
 (segment (start 92.1125 69.0025) (end 93.76 70.65) (width 0.2) (layer "B.Cu") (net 6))
 (segment (start 160.9625 71.0375) (end 160.9625 69.4525) (width 0.2) (layer "B.Cu") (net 6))
 (segment (start 153.8 71.35) (end 160.65 71.35) (width 0.2) (layer "B.Cu") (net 6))
 (segment (start 152.7 70.65) (end 153.1 70.65) (width 0.2) (layer "B.Cu") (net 6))
 (segment (start 174.85 34) (end 174.9 33.95) (width 0.2) (layer "B.Cu") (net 6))
 (segment (start 153.1 70.65) (end 153.8 71.35) (width 0.2) (layer "B.Cu") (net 6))
 (segment (start 166.1 31.25) (end 154.17 31.25) (width 0.2) (layer "F.Cu") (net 17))
 (segment (start 168.65 37.2) (end 168.65 33.8) (width 0.2) (layer "F.Cu") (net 17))
 (segment (start 168.65 33.8) (end 166.1 31.25) (width 0.2) (layer "F.Cu") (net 17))
 (segment (start 154.17 31.25) (end 147.6375 37.7825) (width 0.2) (layer "F.Cu") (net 17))
 (segment (start 169.39125 37.94125) (end 168.65 37.2) (width 0.2) (layer "F.Cu") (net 17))
 (segment (start 171.92625 37.94125) (end 169.39125 37.94125) (width 0.2) (layer "F.Cu") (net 17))
 (segment (start 166.691 40.4821) (end 159.07015 32.86125) (width 0.2) (layer "F.Cu") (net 9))
 (segment (start 100.965 76.04125) (end 100.965 81.9146) (width 0.2) (layer "F.Cu") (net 9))
 (segment (start 158.35645 83.3455) (end 166.691 75.01095) (width 0.2) (layer "F.Cu") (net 9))
 (segment (start 159.07015 32.86125) (end 156.68625 32.86125) (width 0.2) (layer "F.Cu") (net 9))
 (segment (start 100.965 81.9146) (end 102.3959 83.3455) (width 0.2) (layer "F.Cu") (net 9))
 (segment (start 102.3959 83.3455) (end 158.35645 83.3455) (width 0.2) (layer "F.Cu") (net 9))
 (segment (start 166.691 75.01095) (end 166.691 40.4821) (width 0.2) (layer "F.Cu") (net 9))
 (segment (start 120.015 76.04125) (end 121.4463 77.47255) (width 0.2) (layer "F.Cu") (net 12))
 (segment (start 165.50035 73.8203) (end 165.50035 40.4821) (width 0.2) (layer "F.Cu") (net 12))
 (segment (start 160.4195 35.40125) (end 156.68625 35.40125) (width 0.2) (layer "F.Cu") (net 12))
 (segment (start 157.1658 82.15485) (end 165.50035 73.8203) (width 0.2) (layer "F.Cu") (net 12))
 (segment (start 165.50035 40.4821) (end 160.4195 35.40125) (width 0.2) (layer "F.Cu") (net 12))
 (segment (start 121.4463 77.47255) (end 121.4463 82.15485) (width 0.2) (layer "F.Cu") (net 12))
 (segment (start 121.4463 82.15485) (end 157.1658 82.15485) (width 0.2) (layer "F.Cu") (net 12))
 (segment (start 162.08375 76.04125) (end 164.30625 73.81875) (width 0.2) (layer "F.Cu") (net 4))
 (segment (start 164.30625 73.81875) (end 164.30625 40.48125) (width 0.2) (layer "F.Cu") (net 4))
 (segment (start 164.30625 40.48125) (end 161.76625 37.94125) (width 0.2) (layer "F.Cu") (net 4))
 (segment (start 161.76625 37.94125) (end 156.68625 37.94125) (width 0.2) (layer "F.Cu") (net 4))
 (segment (start 139.065 76.04125) (end 162.08375 76.04125) (width 0.2) (layer "F.Cu") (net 4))
 (segment (start 112.9518 56.99125) (end 120.25565 64.2951) (width 0.2) (layer "B.Cu") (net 13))
 (segment (start 155.97515 64.2951) (end 160.73775 59.5325) (width 0.2) (layer "B.Cu") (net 13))
 (segment (start 160.73775 44.53275) (end 156.68625 40.48125) (width 0.2) (layer "B.Cu") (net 13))
 (segment (start 160.73775 59.5325) (end 160.73775 44.53275) (width 0.2) (layer "B.Cu") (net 13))
 (segment (start 100.965 56.99125) (end 112.9518 56.99125) (width 0.2) (layer "B.Cu") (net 13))
 (segment (start 120.25565 64.2951) (end 155.97515 64.2951) (width 0.2) (layer "B.Cu") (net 13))
 (segment (start 132.05875 56.99125) (end 140.94875 48.10125) (width 0.2) (layer "B.Cu") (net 11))
 (segment (start 140.94875 48.10125) (end 156.68625 48.10125) (width 0.2) (layer "B.Cu") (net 11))
 (segment (start 120.015 56.99125) (end 132.05875 56.99125) (width 0.2) (layer "B.Cu") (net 11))
 (segment (start 162.8 51.3) (end 162.75 51.35) (width 0.2) (layer "F.Cu") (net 5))
 (segment (start 158.75 51.35) (end 162.75 51.35) (width 0.2) (layer "F.Cu") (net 5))
 (via (at 162.75 51.35) (size 0.6) (drill 0.3) (layers "F.Cu" "B.Cu") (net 5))
 (via (at 158.75 51.35) (size 0.6) (drill 0.3) (layers "F.Cu" "B.Cu") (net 5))
 (segment (start 162.75 51.35) (end 165.99875 48.10125) (width 0.2) (layer "B.Cu") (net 5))
 (segment (start 165.99875 48.10125) (end 171.92625 48.10125) (width 0.2) (layer "B.Cu") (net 5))
 (segment (start 139.065 56.99125) (end 139.22495 57.1512) (width 0.2) (layer "B.Cu") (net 5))
 (segment (start 158.7 51.3) (end 158.75 51.35) (width 0.2) (layer "B.Cu") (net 5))
 (segment (start 144.75625 51.3) (end 148.3 51.3) (width 0.2) (layer "B.Cu") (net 5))
 (segment (start 148.3 51.3) (end 158.7 51.3) (width 0.2) (layer "B.Cu") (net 5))
 (segment (start 139.065 56.99125) (end 144.75625 51.3) (width 0.2) (layer "B.Cu") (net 5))
 (segment (start 85.45 87.6) (end 84.9 87.05) (width 0.2) (layer "F.Cu") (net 2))
 (segment (start 175.3 45.5) (end 175.3 78.3) (width 0.2) (layer "F.Cu") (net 2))
 (segment (start 85.725 47.925) (end 85.725 42.8625) (width 0.2) (layer "F.Cu") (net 2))
 (segment (start 175.23875 45.56125) (end 175.3 45.5) (width 0.2) (layer "F.Cu") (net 2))
 (segment (start 84.9 87.05) (end 84.9 48.75) (width 0.2) (layer "F.Cu") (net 2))
 (segment (start 166 87.6) (end 85.45 87.6) (width 0.2) (layer "F.Cu") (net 2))
 (segment (start 84.9 48.75) (end 85.725 47.925) (width 0.2) (layer "F.Cu") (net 2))
 (segment (start 175.3 78.3) (end 166 87.6) (width 0.2) (layer "F.Cu") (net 2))
 (segment (start 171.92625 45.56125) (end 175.23875 45.56125) (width 0.2) (layer "F.Cu") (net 2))
 (segment (start 170.4208 43.02125) (end 171.92625 43.02125) (width 0.2) (layer "F.Cu") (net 1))
 (segment (start 169.0723 42.8634) (end 170.26295 42.8634) (width 0.2) (layer "F.Cu") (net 1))
 (segment (start 169.0723 39.29145) (end 169.0723 42.8634) (width 0.2) (layer "F.Cu") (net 1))
 (segment (start 170.26295 42.8634) (end 170.4208 43.02125) (width 0.2) (layer "F.Cu") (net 1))
 (via (at 169.0723 39.29145) (size 0.6) (drill 0.3) (layers "F.Cu" "B.Cu") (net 1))
 (via (at 169.0723 39.29145) (size 0.6) (drill 0.3) (layers "F.Cu" "B.Cu") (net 1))
 (via (at 169.0723 39.29145) (size 0.6) (drill 0.3) (layers "F.Cu" "B.Cu") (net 1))
 (segment (start 85.725 37.8625) (end 85.725 33.34) (width 0.2) (layer "B.Cu") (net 1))
 (segment (start 88.48775 30.57725) (end 169.0723 30.57725) (width 0.2) (layer "B.Cu") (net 1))
 (segment (start 85.725 33.34) (end 88.48775 30.57725) (width 0.2) (layer "B.Cu") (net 1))
 (segment (start 169.0723 30.57725) (end 169.0723 32.14755) (width 0.2) (layer "B.Cu") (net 1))
 (segment (start 169.0723 32.14755) (end 169.0723 39.29145) (width 0.2) (layer "B.Cu") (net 1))
 (segment (start 145.1 40.65) (end 145.1 46.05) (width 0.2) (layer "F.Cu") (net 15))
 (segment (start 152.5 46.05) (end 152.98875 45.56125) (width 0.2) (layer "F.Cu") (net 15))
 (segment (start 145.1 46.05) (end 152.5 46.05) (width 0.2) (layer "F.Cu") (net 15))
 (segment (start 145.4275 40.3225) (end 145.1 40.65) (width 0.2) (layer "F.Cu") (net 15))
 (segment (start 147.6375 40.3225) (end 145.4275 40.3225) (width 0.2) (layer "F.Cu") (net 15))
 (segment (start 152.98875 45.56125) (end 155.85125 45.56125) (width 0.2) (layer "F.Cu") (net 15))
 (segment (start 147.6375 42.8625) (end 156.5275 42.8625) (width 0.2) (layer "F.Cu") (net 14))
 (segment (start 156.5275 42.8625) (end 156.68625 43.02125) (width 0.2) (layer "F.Cu") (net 14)))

